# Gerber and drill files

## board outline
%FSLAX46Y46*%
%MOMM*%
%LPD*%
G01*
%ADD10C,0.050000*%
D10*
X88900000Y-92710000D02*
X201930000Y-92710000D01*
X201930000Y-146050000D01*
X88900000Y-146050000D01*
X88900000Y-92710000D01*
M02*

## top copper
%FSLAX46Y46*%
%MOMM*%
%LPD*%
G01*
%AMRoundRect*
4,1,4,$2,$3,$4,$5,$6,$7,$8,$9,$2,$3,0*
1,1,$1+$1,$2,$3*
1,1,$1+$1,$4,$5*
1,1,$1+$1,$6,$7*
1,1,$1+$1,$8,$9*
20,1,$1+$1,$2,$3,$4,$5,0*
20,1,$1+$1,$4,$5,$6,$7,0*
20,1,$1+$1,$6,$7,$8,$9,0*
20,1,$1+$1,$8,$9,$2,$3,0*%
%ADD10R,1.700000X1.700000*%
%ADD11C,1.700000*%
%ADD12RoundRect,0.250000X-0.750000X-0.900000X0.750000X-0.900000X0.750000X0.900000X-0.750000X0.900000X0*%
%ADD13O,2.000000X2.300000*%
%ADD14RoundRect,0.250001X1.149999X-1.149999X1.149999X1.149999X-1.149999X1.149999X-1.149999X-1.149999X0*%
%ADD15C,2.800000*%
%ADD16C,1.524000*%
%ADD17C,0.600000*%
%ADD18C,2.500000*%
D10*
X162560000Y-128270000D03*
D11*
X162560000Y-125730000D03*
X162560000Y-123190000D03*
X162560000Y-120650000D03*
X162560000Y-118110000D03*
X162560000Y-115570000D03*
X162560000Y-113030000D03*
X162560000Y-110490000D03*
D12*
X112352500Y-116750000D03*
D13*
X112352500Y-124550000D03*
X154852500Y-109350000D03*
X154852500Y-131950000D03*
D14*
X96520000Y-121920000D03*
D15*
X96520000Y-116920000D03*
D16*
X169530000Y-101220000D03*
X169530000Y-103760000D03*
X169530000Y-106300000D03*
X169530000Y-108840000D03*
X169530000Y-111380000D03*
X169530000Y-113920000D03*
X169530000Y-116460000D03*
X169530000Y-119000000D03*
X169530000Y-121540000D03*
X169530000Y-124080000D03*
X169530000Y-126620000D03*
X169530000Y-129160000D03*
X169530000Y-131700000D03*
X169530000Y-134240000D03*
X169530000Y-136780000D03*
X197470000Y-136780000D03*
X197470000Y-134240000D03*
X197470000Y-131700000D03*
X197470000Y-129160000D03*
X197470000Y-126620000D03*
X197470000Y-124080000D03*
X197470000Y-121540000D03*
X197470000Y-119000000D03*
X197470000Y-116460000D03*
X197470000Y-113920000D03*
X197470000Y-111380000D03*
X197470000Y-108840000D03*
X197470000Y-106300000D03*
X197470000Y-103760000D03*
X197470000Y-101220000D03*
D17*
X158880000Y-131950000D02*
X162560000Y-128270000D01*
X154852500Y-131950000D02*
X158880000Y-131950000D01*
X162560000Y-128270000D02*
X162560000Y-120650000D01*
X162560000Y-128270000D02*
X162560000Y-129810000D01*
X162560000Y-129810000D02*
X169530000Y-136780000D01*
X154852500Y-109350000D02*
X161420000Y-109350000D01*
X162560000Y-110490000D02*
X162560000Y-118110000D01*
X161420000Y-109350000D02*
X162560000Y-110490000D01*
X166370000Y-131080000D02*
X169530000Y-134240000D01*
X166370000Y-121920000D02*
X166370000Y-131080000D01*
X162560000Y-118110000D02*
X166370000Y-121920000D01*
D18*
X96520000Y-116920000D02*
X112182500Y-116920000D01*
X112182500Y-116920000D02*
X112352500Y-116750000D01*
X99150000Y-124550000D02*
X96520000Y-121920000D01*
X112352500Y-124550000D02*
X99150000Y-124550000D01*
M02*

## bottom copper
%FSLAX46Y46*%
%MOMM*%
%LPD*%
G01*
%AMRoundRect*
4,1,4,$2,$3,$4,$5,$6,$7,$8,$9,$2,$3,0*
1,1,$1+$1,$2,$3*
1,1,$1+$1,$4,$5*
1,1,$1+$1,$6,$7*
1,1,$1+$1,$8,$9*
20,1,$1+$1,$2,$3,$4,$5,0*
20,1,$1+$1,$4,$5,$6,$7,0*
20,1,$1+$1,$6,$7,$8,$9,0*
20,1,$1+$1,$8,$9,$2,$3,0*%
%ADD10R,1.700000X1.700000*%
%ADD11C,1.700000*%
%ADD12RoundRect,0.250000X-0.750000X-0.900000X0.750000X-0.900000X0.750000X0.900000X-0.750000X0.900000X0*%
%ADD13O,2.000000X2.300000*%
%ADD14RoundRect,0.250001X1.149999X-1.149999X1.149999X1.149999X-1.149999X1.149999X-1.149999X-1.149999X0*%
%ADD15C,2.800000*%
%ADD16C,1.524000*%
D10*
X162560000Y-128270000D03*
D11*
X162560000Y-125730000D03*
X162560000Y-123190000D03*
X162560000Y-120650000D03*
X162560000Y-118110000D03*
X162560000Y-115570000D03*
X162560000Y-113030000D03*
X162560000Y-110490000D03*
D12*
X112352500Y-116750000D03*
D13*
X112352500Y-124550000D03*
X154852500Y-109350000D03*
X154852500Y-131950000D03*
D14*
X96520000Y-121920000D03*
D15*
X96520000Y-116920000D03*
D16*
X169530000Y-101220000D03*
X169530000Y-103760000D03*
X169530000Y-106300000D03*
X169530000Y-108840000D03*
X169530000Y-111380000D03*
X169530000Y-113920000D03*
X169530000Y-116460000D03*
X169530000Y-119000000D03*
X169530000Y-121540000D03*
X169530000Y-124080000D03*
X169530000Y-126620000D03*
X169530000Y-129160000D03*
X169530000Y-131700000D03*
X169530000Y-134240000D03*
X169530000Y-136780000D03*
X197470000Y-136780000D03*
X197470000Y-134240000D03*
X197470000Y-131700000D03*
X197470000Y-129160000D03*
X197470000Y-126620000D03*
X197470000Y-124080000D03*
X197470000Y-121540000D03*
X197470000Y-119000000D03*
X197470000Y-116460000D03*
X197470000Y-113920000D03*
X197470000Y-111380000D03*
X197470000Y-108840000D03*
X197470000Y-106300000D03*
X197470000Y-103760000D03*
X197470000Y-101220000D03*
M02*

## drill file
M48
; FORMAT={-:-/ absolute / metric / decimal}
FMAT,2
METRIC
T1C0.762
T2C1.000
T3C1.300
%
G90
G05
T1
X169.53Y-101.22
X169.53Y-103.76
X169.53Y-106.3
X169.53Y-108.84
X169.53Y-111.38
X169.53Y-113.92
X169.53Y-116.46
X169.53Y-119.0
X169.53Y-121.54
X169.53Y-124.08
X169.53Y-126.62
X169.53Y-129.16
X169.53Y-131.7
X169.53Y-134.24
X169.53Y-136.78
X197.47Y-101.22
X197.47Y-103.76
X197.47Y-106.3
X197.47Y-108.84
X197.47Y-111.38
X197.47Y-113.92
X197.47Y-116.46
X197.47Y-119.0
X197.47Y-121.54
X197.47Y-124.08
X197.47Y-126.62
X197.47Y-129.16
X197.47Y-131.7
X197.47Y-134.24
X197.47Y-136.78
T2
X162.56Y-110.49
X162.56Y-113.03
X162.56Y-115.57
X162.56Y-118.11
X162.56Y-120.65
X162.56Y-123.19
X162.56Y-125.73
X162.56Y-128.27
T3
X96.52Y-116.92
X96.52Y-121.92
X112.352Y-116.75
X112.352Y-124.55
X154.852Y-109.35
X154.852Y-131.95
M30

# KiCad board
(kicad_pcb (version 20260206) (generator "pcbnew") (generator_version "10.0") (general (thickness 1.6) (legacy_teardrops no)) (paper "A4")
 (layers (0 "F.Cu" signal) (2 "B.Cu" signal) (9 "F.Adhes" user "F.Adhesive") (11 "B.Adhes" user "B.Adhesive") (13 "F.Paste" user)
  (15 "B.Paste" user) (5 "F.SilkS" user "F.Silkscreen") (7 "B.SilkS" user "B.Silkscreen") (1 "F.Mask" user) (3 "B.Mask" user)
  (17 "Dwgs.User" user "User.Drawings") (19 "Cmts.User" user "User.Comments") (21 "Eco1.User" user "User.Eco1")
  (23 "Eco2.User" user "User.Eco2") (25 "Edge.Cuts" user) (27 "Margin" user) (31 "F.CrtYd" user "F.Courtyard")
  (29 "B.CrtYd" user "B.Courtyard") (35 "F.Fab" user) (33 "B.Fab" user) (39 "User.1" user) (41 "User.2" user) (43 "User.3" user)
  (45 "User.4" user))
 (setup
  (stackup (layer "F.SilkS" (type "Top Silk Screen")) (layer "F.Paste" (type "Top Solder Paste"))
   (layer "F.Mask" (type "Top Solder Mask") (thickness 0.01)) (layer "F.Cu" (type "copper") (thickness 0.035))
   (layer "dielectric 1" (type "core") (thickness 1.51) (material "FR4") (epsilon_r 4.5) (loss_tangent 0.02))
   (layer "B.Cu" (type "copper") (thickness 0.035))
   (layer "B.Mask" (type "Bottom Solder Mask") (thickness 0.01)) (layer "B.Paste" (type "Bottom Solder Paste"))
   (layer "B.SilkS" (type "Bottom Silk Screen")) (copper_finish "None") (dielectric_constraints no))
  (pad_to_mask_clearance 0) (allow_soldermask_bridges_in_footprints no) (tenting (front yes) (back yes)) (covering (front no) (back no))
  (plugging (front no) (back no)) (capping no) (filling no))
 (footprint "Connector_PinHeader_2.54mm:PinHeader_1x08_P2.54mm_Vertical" (layer "F.Cu") (at 162.56 128.27 180)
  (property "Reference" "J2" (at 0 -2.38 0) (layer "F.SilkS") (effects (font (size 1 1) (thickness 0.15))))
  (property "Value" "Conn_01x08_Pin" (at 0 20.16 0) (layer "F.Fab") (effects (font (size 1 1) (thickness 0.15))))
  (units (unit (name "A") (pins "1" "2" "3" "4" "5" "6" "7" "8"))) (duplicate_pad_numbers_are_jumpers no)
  (pad "1" thru_hole rect (at 0 0 180) (size 1.7 1.7) (drill 1) (layers "*.Cu" "*.Mask") (remove_unused_layers no) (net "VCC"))
  (pad "2" thru_hole circle (at 0 2.54 180) (size 1.7 1.7) (drill 1) (layers "*.Cu" "*.Mask") (remove_unused_layers no) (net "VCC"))
  (pad "3" thru_hole circle (at 0 5.08 180) (size 1.7 1.7) (drill 1) (layers "*.Cu" "*.Mask") (remove_unused_layers no) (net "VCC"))
  (pad "4" thru_hole circle (at 0 7.62 180) (size 1.7 1.7) (drill 1) (layers "*.Cu" "*.Mask") (remove_unused_layers no) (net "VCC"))
  (pad "5" thru_hole circle (at 0 10.16 180) (size 1.7 1.7) (drill 1) (layers "*.Cu" "*.Mask") (remove_unused_layers no) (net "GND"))
  (pad "6" thru_hole circle (at 0 12.7 180) (size 1.7 1.7) (drill 1) (layers "*.Cu" "*.Mask") (remove_unused_layers no) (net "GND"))
  (pad "7" thru_hole circle (at 0 15.24 180) (size 1.7 1.7) (drill 1) (layers "*.Cu" "*.Mask") (remove_unused_layers no) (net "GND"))
  (pad "8" thru_hole circle (at 0 17.78 180) (size 1.7 1.7) (drill 1) (layers "*.Cu" "*.Mask") (remove_unused_layers no) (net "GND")))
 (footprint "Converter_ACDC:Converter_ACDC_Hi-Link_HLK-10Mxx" (layer "F.Cu") (at 112.3525 116.75)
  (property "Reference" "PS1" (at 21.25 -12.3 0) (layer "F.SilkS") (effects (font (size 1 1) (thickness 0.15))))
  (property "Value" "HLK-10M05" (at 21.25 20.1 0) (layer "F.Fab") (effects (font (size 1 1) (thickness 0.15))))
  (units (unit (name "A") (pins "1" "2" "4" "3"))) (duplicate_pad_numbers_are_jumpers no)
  (pad "1" thru_hole roundrect (at 0 0) (size 2 2.3) (drill 1.3) (layers "*.Cu" "*.Mask") (remove_unused_layers no) (roundrect_rratio 0.125)
   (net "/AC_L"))
  (pad "2" thru_hole oval (at 0 7.8) (size 2 2.3) (drill 1.3) (layers "*.Cu" "*.Mask") (remove_unused_layers no) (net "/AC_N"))
  (pad "3" thru_hole oval (at 42.5 -7.4) (size 2 2.3) (drill 1.3) (layers "*.Cu" "*.Mask") (remove_unused_layers no) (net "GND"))
  (pad "4" thru_hole oval (at 42.5 15.2) (size 2 2.3) (drill 1.3) (layers "*.Cu" "*.Mask") (remove_unused_layers no) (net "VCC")))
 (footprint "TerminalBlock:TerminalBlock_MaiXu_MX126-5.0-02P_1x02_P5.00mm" (layer "F.Cu") (at 96.52 121.92 90)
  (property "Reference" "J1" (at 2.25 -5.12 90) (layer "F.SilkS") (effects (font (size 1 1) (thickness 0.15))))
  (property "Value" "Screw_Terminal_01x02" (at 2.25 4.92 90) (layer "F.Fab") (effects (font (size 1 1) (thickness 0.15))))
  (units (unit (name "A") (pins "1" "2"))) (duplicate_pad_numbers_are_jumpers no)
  (pad "1" thru_hole roundrect (at 0 0 90) (size 2.8 2.8) (drill 1.3) (layers "*.Cu" "*.Mask") (remove_unused_layers no)
   (roundrect_rratio 0.089286) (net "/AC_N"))
  (pad "2" thru_hole circle (at 5 0 90) (size 2.8 2.8) (drill 1.3) (layers "*.Cu" "*.Mask") (remove_unused_layers no) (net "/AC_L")))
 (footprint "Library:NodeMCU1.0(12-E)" (layer "F.Cu") (at 183.5 119)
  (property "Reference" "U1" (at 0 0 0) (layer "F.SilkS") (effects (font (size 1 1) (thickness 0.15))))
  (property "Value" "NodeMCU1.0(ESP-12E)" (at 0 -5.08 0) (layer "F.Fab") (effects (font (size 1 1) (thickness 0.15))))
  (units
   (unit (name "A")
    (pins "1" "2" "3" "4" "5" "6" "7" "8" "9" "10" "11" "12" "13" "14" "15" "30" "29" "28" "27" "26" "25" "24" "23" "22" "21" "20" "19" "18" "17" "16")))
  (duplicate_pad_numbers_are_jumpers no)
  (pad "1" thru_hole circle (at -13.97 -17.78) (size 1.524 1.524) (drill 0.762) (layers "*.Cu" "*.Mask" "F.SilkS") (remove_unused_layers no)
   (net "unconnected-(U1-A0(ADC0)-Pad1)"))
  (pad "2" thru_hole circle (at -13.97 -15.24) (size 1.524 1.524) (drill 0.762) (layers "*.Cu" "*.Mask" "F.SilkS") (remove_unused_layers no)
   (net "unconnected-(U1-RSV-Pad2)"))
  (pad "3" thru_hole circle (at -13.97 -12.7) (size 1.524 1.524) (drill 0.762) (layers "*.Cu" "*.Mask" "F.SilkS") (remove_unused_layers no)
   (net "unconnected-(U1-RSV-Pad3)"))
  (pad "4" thru_hole circle (at -13.97 -10.16) (size 1.524 1.524) (drill 0.762) (layers "*.Cu" "*.Mask" "F.SilkS") (remove_unused_layers no)
   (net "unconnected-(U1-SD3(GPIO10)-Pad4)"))
  (pad "5" thru_hole circle (at -13.97 -7.62) (size 1.524 1.524) (drill 0.762) (layers "*.Cu" "*.Mask" "F.SilkS") (remove_unused_layers no)
   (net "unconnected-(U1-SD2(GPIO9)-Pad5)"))
  (pad "6" thru_hole circle (at -13.97 -5.08) (size 1.524 1.524) (drill 0.762) (layers "*.Cu" "*.Mask" "F.SilkS") (remove_unused_layers no)
   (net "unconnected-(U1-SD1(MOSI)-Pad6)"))
  (pad "7" thru_hole circle (at -13.97 -2.54) (size 1.524 1.524) (drill 0.762) (layers "*.Cu" "*.Mask" "F.SilkS") (remove_unused_layers no)
   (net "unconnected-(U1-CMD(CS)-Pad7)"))
  (pad "8" thru_hole circle (at -13.97 0) (size 1.524 1.524) (drill 0.762) (layers "*.Cu" "*.Mask" "F.SilkS") (remove_unused_layers no)
   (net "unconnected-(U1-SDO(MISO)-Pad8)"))
  (pad "9" thru_hole circle (at -13.97 2.54) (size 1.524 1.524) (drill 0.762) (layers "*.Cu" "*.Mask" "F.SilkS") (remove_unused_layers no)
   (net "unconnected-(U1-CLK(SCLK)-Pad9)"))
  (pad "10" thru_hole circle (at -13.97 5.08) (size 1.524 1.524) (drill 0.762) (layers "*.Cu" "*.Mask" "F.SilkS") (remove_unused_layers no)
   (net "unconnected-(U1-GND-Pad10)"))
  (pad "11" thru_hole circle (at -13.97 7.62) (size 1.524 1.524) (drill 0.762) (layers "*.Cu" "*.Mask" "F.SilkS") (remove_unused_layers no)
   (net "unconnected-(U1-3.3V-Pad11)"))
  (pad "12" thru_hole circle (at -13.97 10.16) (size 1.524 1.524) (drill 0.762) (layers "*.Cu" "*.Mask" "F.SilkS") (remove_unused_layers no)
   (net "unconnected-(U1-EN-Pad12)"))
  (pad "13" thru_hole circle (at -13.97 12.7) (size 1.524 1.524) (drill 0.762) (layers "*.Cu" "*.Mask" "F.SilkS") (remove_unused_layers no)
   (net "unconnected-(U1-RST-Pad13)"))
  (pad "14" thru_hole circle (at -13.97 15.24) (size 1.524 1.524) (drill 0.762) (layers "*.Cu" "*.Mask" "F.SilkS") (remove_unused_layers no)
   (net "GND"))
  (pad "15" thru_hole circle (at -13.97 17.78) (size 1.524 1.524) (drill 0.762) (layers "*.Cu" "*.Mask" "F.SilkS") (remove_unused_layers no)
   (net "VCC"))
  (pad "16" thru_hole circle (at 13.97 17.78) (size 1.524 1.524) (drill 0.762) (layers "*.Cu" "*.Mask" "F.SilkS") (remove_unused_layers no)
   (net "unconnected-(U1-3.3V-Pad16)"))
  (pad "17" thru_hole circle (at 13.97 15.24) (size 1.524 1.524) (drill 0.762) (layers "*.Cu" "*.Mask" "F.SilkS") (remove_unused_layers no)
   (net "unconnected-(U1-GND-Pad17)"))
  (pad "18" thru_hole circle (at 13.97 12.7) (size 1.524 1.524) (drill 0.762) (layers "*.Cu" "*.Mask" "F.SilkS") (remove_unused_layers no)
   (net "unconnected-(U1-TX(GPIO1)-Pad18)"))
  (pad "19" thru_hole circle (at 13.97 10.16) (size 1.524 1.524) (drill 0.762) (layers "*.Cu" "*.Mask" "F.SilkS") (remove_unused_layers no)
   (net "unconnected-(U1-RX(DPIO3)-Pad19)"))
  (pad "20" thru_hole circle (at 13.97 7.62) (size 1.524 1.524) (drill 0.762) (layers "*.Cu" "*.Mask" "F.SilkS") (remove_unused_layers no)
   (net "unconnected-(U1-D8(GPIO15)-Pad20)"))
  (pad "21" thru_hole circle (at 13.97 5.08) (size 1.524 1.524) (drill 0.762) (layers "*.Cu" "*.Mask" "F.SilkS") (remove_unused_layers no)
   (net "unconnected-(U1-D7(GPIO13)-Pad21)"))
  (pad "22" thru_hole circle (at 13.97 2.54) (size 1.524 1.524) (drill 0.762) (layers "*.Cu" "*.Mask" "F.SilkS") (remove_unused_layers no)
   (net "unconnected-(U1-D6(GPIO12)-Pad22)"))
  (pad "23" thru_hole circle (at 13.97 0) (size 1.524 1.524) (drill 0.762) (layers "*.Cu" "*.Mask" "F.SilkS") (remove_unused_layers no)
   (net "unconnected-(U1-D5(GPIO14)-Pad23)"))
  (pad "24" thru_hole circle (at 13.97 -2.54) (size 1.524 1.524) (drill 0.762) (layers "*.Cu" "*.Mask" "F.SilkS") (remove_unused_layers no)
   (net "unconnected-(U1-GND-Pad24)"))
  (pad "25" thru_hole circle (at 13.97 -5.08) (size 1.524 1.524) (drill 0.762) (layers "*.Cu" "*.Mask" "F.SilkS") (remove_unused_layers no)
   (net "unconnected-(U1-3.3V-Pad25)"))
  (pad "26" thru_hole circle (at 13.97 -7.62) (size 1.524 1.524) (drill 0.762) (layers "*.Cu" "*.Mask" "F.SilkS") (remove_unused_layers no)
   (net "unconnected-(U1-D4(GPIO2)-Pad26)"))
  (pad "27" thru_hole circle (at 13.97 -10.16) (size 1.524 1.524) (drill 0.762) (layers "*.Cu" "*.Mask" "F.SilkS") (remove_unused_layers no)
   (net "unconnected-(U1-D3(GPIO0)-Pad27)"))
  (pad "28" thru_hole circle (at 13.97 -12.7) (size 1.524 1.524) (drill 0.762) (layers "*.Cu" "*.Mask" "F.SilkS") (remove_unused_layers no)
   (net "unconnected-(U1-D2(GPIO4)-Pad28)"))
  (pad "29" thru_hole circle (at 13.97 -15.24) (size 1.524 1.524) (drill 0.762) (layers "*.Cu" "*.Mask" "F.SilkS") (remove_unused_layers no)
   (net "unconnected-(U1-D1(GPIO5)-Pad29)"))
  (pad "30" thru_hole circle (at 13.97 -17.78) (size 1.524 1.524) (drill 0.762) (layers "*.Cu" "*.Mask" "F.SilkS") (remove_unused_layers no)
   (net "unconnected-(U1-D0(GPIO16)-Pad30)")))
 (gr_rect (start 88.9 92.71) (end 201.93 146.05) (stroke (width 0.05) (type default)) (fill no) (layer "Edge.Cuts"))
 (segment (start 158.88 131.95) (end 162.56 128.27) (width 0.6) (layer "F.Cu") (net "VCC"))
 (segment (start 154.8525 131.95) (end 158.88 131.95) (width 0.6) (layer "F.Cu") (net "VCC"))
 (segment (start 162.56 128.27) (end 162.56 120.65) (width 0.6) (layer "F.Cu") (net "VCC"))
 (segment (start 162.56 128.27) (end 162.56 129.81) (width 0.6) (layer "F.Cu") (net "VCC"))
 (segment (start 162.56 129.81) (end 169.53 136.78) (width 0.6) (layer "F.Cu") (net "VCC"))
 (segment (start 154.8525 109.35) (end 161.42 109.35) (width 0.6) (layer "F.Cu") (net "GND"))
 (segment (start 162.56 110.49) (end 162.56 118.11) (width 0.6) (layer "F.Cu") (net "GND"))
 (segment (start 161.42 109.35) (end 162.56 110.49) (width 0.6) (layer "F.Cu") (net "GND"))
 (segment (start 166.37 131.08) (end 169.53 134.24) (width 0.6) (layer "F.Cu") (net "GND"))
 (segment (start 166.37 121.92) (end 166.37 131.08) (width 0.6) (layer "F.Cu") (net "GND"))
 (segment (start 162.56 118.11) (end 166.37 121.92) (width 0.6) (layer "F.Cu") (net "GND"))
 (segment (start 96.52 116.92) (end 112.1825 116.92) (width 2.5) (layer "F.Cu") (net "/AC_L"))
 (segment (start 112.1825 116.92) (end 112.3525 116.75) (width 2.5) (layer "F.Cu") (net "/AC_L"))
 (segment (start 99.15 124.55) (end 96.52 121.92) (width 2.5) (layer "F.Cu") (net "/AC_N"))
 (segment (start 112.3525 124.55) (end 99.15 124.55) (width 2.5) (layer "F.Cu") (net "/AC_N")))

